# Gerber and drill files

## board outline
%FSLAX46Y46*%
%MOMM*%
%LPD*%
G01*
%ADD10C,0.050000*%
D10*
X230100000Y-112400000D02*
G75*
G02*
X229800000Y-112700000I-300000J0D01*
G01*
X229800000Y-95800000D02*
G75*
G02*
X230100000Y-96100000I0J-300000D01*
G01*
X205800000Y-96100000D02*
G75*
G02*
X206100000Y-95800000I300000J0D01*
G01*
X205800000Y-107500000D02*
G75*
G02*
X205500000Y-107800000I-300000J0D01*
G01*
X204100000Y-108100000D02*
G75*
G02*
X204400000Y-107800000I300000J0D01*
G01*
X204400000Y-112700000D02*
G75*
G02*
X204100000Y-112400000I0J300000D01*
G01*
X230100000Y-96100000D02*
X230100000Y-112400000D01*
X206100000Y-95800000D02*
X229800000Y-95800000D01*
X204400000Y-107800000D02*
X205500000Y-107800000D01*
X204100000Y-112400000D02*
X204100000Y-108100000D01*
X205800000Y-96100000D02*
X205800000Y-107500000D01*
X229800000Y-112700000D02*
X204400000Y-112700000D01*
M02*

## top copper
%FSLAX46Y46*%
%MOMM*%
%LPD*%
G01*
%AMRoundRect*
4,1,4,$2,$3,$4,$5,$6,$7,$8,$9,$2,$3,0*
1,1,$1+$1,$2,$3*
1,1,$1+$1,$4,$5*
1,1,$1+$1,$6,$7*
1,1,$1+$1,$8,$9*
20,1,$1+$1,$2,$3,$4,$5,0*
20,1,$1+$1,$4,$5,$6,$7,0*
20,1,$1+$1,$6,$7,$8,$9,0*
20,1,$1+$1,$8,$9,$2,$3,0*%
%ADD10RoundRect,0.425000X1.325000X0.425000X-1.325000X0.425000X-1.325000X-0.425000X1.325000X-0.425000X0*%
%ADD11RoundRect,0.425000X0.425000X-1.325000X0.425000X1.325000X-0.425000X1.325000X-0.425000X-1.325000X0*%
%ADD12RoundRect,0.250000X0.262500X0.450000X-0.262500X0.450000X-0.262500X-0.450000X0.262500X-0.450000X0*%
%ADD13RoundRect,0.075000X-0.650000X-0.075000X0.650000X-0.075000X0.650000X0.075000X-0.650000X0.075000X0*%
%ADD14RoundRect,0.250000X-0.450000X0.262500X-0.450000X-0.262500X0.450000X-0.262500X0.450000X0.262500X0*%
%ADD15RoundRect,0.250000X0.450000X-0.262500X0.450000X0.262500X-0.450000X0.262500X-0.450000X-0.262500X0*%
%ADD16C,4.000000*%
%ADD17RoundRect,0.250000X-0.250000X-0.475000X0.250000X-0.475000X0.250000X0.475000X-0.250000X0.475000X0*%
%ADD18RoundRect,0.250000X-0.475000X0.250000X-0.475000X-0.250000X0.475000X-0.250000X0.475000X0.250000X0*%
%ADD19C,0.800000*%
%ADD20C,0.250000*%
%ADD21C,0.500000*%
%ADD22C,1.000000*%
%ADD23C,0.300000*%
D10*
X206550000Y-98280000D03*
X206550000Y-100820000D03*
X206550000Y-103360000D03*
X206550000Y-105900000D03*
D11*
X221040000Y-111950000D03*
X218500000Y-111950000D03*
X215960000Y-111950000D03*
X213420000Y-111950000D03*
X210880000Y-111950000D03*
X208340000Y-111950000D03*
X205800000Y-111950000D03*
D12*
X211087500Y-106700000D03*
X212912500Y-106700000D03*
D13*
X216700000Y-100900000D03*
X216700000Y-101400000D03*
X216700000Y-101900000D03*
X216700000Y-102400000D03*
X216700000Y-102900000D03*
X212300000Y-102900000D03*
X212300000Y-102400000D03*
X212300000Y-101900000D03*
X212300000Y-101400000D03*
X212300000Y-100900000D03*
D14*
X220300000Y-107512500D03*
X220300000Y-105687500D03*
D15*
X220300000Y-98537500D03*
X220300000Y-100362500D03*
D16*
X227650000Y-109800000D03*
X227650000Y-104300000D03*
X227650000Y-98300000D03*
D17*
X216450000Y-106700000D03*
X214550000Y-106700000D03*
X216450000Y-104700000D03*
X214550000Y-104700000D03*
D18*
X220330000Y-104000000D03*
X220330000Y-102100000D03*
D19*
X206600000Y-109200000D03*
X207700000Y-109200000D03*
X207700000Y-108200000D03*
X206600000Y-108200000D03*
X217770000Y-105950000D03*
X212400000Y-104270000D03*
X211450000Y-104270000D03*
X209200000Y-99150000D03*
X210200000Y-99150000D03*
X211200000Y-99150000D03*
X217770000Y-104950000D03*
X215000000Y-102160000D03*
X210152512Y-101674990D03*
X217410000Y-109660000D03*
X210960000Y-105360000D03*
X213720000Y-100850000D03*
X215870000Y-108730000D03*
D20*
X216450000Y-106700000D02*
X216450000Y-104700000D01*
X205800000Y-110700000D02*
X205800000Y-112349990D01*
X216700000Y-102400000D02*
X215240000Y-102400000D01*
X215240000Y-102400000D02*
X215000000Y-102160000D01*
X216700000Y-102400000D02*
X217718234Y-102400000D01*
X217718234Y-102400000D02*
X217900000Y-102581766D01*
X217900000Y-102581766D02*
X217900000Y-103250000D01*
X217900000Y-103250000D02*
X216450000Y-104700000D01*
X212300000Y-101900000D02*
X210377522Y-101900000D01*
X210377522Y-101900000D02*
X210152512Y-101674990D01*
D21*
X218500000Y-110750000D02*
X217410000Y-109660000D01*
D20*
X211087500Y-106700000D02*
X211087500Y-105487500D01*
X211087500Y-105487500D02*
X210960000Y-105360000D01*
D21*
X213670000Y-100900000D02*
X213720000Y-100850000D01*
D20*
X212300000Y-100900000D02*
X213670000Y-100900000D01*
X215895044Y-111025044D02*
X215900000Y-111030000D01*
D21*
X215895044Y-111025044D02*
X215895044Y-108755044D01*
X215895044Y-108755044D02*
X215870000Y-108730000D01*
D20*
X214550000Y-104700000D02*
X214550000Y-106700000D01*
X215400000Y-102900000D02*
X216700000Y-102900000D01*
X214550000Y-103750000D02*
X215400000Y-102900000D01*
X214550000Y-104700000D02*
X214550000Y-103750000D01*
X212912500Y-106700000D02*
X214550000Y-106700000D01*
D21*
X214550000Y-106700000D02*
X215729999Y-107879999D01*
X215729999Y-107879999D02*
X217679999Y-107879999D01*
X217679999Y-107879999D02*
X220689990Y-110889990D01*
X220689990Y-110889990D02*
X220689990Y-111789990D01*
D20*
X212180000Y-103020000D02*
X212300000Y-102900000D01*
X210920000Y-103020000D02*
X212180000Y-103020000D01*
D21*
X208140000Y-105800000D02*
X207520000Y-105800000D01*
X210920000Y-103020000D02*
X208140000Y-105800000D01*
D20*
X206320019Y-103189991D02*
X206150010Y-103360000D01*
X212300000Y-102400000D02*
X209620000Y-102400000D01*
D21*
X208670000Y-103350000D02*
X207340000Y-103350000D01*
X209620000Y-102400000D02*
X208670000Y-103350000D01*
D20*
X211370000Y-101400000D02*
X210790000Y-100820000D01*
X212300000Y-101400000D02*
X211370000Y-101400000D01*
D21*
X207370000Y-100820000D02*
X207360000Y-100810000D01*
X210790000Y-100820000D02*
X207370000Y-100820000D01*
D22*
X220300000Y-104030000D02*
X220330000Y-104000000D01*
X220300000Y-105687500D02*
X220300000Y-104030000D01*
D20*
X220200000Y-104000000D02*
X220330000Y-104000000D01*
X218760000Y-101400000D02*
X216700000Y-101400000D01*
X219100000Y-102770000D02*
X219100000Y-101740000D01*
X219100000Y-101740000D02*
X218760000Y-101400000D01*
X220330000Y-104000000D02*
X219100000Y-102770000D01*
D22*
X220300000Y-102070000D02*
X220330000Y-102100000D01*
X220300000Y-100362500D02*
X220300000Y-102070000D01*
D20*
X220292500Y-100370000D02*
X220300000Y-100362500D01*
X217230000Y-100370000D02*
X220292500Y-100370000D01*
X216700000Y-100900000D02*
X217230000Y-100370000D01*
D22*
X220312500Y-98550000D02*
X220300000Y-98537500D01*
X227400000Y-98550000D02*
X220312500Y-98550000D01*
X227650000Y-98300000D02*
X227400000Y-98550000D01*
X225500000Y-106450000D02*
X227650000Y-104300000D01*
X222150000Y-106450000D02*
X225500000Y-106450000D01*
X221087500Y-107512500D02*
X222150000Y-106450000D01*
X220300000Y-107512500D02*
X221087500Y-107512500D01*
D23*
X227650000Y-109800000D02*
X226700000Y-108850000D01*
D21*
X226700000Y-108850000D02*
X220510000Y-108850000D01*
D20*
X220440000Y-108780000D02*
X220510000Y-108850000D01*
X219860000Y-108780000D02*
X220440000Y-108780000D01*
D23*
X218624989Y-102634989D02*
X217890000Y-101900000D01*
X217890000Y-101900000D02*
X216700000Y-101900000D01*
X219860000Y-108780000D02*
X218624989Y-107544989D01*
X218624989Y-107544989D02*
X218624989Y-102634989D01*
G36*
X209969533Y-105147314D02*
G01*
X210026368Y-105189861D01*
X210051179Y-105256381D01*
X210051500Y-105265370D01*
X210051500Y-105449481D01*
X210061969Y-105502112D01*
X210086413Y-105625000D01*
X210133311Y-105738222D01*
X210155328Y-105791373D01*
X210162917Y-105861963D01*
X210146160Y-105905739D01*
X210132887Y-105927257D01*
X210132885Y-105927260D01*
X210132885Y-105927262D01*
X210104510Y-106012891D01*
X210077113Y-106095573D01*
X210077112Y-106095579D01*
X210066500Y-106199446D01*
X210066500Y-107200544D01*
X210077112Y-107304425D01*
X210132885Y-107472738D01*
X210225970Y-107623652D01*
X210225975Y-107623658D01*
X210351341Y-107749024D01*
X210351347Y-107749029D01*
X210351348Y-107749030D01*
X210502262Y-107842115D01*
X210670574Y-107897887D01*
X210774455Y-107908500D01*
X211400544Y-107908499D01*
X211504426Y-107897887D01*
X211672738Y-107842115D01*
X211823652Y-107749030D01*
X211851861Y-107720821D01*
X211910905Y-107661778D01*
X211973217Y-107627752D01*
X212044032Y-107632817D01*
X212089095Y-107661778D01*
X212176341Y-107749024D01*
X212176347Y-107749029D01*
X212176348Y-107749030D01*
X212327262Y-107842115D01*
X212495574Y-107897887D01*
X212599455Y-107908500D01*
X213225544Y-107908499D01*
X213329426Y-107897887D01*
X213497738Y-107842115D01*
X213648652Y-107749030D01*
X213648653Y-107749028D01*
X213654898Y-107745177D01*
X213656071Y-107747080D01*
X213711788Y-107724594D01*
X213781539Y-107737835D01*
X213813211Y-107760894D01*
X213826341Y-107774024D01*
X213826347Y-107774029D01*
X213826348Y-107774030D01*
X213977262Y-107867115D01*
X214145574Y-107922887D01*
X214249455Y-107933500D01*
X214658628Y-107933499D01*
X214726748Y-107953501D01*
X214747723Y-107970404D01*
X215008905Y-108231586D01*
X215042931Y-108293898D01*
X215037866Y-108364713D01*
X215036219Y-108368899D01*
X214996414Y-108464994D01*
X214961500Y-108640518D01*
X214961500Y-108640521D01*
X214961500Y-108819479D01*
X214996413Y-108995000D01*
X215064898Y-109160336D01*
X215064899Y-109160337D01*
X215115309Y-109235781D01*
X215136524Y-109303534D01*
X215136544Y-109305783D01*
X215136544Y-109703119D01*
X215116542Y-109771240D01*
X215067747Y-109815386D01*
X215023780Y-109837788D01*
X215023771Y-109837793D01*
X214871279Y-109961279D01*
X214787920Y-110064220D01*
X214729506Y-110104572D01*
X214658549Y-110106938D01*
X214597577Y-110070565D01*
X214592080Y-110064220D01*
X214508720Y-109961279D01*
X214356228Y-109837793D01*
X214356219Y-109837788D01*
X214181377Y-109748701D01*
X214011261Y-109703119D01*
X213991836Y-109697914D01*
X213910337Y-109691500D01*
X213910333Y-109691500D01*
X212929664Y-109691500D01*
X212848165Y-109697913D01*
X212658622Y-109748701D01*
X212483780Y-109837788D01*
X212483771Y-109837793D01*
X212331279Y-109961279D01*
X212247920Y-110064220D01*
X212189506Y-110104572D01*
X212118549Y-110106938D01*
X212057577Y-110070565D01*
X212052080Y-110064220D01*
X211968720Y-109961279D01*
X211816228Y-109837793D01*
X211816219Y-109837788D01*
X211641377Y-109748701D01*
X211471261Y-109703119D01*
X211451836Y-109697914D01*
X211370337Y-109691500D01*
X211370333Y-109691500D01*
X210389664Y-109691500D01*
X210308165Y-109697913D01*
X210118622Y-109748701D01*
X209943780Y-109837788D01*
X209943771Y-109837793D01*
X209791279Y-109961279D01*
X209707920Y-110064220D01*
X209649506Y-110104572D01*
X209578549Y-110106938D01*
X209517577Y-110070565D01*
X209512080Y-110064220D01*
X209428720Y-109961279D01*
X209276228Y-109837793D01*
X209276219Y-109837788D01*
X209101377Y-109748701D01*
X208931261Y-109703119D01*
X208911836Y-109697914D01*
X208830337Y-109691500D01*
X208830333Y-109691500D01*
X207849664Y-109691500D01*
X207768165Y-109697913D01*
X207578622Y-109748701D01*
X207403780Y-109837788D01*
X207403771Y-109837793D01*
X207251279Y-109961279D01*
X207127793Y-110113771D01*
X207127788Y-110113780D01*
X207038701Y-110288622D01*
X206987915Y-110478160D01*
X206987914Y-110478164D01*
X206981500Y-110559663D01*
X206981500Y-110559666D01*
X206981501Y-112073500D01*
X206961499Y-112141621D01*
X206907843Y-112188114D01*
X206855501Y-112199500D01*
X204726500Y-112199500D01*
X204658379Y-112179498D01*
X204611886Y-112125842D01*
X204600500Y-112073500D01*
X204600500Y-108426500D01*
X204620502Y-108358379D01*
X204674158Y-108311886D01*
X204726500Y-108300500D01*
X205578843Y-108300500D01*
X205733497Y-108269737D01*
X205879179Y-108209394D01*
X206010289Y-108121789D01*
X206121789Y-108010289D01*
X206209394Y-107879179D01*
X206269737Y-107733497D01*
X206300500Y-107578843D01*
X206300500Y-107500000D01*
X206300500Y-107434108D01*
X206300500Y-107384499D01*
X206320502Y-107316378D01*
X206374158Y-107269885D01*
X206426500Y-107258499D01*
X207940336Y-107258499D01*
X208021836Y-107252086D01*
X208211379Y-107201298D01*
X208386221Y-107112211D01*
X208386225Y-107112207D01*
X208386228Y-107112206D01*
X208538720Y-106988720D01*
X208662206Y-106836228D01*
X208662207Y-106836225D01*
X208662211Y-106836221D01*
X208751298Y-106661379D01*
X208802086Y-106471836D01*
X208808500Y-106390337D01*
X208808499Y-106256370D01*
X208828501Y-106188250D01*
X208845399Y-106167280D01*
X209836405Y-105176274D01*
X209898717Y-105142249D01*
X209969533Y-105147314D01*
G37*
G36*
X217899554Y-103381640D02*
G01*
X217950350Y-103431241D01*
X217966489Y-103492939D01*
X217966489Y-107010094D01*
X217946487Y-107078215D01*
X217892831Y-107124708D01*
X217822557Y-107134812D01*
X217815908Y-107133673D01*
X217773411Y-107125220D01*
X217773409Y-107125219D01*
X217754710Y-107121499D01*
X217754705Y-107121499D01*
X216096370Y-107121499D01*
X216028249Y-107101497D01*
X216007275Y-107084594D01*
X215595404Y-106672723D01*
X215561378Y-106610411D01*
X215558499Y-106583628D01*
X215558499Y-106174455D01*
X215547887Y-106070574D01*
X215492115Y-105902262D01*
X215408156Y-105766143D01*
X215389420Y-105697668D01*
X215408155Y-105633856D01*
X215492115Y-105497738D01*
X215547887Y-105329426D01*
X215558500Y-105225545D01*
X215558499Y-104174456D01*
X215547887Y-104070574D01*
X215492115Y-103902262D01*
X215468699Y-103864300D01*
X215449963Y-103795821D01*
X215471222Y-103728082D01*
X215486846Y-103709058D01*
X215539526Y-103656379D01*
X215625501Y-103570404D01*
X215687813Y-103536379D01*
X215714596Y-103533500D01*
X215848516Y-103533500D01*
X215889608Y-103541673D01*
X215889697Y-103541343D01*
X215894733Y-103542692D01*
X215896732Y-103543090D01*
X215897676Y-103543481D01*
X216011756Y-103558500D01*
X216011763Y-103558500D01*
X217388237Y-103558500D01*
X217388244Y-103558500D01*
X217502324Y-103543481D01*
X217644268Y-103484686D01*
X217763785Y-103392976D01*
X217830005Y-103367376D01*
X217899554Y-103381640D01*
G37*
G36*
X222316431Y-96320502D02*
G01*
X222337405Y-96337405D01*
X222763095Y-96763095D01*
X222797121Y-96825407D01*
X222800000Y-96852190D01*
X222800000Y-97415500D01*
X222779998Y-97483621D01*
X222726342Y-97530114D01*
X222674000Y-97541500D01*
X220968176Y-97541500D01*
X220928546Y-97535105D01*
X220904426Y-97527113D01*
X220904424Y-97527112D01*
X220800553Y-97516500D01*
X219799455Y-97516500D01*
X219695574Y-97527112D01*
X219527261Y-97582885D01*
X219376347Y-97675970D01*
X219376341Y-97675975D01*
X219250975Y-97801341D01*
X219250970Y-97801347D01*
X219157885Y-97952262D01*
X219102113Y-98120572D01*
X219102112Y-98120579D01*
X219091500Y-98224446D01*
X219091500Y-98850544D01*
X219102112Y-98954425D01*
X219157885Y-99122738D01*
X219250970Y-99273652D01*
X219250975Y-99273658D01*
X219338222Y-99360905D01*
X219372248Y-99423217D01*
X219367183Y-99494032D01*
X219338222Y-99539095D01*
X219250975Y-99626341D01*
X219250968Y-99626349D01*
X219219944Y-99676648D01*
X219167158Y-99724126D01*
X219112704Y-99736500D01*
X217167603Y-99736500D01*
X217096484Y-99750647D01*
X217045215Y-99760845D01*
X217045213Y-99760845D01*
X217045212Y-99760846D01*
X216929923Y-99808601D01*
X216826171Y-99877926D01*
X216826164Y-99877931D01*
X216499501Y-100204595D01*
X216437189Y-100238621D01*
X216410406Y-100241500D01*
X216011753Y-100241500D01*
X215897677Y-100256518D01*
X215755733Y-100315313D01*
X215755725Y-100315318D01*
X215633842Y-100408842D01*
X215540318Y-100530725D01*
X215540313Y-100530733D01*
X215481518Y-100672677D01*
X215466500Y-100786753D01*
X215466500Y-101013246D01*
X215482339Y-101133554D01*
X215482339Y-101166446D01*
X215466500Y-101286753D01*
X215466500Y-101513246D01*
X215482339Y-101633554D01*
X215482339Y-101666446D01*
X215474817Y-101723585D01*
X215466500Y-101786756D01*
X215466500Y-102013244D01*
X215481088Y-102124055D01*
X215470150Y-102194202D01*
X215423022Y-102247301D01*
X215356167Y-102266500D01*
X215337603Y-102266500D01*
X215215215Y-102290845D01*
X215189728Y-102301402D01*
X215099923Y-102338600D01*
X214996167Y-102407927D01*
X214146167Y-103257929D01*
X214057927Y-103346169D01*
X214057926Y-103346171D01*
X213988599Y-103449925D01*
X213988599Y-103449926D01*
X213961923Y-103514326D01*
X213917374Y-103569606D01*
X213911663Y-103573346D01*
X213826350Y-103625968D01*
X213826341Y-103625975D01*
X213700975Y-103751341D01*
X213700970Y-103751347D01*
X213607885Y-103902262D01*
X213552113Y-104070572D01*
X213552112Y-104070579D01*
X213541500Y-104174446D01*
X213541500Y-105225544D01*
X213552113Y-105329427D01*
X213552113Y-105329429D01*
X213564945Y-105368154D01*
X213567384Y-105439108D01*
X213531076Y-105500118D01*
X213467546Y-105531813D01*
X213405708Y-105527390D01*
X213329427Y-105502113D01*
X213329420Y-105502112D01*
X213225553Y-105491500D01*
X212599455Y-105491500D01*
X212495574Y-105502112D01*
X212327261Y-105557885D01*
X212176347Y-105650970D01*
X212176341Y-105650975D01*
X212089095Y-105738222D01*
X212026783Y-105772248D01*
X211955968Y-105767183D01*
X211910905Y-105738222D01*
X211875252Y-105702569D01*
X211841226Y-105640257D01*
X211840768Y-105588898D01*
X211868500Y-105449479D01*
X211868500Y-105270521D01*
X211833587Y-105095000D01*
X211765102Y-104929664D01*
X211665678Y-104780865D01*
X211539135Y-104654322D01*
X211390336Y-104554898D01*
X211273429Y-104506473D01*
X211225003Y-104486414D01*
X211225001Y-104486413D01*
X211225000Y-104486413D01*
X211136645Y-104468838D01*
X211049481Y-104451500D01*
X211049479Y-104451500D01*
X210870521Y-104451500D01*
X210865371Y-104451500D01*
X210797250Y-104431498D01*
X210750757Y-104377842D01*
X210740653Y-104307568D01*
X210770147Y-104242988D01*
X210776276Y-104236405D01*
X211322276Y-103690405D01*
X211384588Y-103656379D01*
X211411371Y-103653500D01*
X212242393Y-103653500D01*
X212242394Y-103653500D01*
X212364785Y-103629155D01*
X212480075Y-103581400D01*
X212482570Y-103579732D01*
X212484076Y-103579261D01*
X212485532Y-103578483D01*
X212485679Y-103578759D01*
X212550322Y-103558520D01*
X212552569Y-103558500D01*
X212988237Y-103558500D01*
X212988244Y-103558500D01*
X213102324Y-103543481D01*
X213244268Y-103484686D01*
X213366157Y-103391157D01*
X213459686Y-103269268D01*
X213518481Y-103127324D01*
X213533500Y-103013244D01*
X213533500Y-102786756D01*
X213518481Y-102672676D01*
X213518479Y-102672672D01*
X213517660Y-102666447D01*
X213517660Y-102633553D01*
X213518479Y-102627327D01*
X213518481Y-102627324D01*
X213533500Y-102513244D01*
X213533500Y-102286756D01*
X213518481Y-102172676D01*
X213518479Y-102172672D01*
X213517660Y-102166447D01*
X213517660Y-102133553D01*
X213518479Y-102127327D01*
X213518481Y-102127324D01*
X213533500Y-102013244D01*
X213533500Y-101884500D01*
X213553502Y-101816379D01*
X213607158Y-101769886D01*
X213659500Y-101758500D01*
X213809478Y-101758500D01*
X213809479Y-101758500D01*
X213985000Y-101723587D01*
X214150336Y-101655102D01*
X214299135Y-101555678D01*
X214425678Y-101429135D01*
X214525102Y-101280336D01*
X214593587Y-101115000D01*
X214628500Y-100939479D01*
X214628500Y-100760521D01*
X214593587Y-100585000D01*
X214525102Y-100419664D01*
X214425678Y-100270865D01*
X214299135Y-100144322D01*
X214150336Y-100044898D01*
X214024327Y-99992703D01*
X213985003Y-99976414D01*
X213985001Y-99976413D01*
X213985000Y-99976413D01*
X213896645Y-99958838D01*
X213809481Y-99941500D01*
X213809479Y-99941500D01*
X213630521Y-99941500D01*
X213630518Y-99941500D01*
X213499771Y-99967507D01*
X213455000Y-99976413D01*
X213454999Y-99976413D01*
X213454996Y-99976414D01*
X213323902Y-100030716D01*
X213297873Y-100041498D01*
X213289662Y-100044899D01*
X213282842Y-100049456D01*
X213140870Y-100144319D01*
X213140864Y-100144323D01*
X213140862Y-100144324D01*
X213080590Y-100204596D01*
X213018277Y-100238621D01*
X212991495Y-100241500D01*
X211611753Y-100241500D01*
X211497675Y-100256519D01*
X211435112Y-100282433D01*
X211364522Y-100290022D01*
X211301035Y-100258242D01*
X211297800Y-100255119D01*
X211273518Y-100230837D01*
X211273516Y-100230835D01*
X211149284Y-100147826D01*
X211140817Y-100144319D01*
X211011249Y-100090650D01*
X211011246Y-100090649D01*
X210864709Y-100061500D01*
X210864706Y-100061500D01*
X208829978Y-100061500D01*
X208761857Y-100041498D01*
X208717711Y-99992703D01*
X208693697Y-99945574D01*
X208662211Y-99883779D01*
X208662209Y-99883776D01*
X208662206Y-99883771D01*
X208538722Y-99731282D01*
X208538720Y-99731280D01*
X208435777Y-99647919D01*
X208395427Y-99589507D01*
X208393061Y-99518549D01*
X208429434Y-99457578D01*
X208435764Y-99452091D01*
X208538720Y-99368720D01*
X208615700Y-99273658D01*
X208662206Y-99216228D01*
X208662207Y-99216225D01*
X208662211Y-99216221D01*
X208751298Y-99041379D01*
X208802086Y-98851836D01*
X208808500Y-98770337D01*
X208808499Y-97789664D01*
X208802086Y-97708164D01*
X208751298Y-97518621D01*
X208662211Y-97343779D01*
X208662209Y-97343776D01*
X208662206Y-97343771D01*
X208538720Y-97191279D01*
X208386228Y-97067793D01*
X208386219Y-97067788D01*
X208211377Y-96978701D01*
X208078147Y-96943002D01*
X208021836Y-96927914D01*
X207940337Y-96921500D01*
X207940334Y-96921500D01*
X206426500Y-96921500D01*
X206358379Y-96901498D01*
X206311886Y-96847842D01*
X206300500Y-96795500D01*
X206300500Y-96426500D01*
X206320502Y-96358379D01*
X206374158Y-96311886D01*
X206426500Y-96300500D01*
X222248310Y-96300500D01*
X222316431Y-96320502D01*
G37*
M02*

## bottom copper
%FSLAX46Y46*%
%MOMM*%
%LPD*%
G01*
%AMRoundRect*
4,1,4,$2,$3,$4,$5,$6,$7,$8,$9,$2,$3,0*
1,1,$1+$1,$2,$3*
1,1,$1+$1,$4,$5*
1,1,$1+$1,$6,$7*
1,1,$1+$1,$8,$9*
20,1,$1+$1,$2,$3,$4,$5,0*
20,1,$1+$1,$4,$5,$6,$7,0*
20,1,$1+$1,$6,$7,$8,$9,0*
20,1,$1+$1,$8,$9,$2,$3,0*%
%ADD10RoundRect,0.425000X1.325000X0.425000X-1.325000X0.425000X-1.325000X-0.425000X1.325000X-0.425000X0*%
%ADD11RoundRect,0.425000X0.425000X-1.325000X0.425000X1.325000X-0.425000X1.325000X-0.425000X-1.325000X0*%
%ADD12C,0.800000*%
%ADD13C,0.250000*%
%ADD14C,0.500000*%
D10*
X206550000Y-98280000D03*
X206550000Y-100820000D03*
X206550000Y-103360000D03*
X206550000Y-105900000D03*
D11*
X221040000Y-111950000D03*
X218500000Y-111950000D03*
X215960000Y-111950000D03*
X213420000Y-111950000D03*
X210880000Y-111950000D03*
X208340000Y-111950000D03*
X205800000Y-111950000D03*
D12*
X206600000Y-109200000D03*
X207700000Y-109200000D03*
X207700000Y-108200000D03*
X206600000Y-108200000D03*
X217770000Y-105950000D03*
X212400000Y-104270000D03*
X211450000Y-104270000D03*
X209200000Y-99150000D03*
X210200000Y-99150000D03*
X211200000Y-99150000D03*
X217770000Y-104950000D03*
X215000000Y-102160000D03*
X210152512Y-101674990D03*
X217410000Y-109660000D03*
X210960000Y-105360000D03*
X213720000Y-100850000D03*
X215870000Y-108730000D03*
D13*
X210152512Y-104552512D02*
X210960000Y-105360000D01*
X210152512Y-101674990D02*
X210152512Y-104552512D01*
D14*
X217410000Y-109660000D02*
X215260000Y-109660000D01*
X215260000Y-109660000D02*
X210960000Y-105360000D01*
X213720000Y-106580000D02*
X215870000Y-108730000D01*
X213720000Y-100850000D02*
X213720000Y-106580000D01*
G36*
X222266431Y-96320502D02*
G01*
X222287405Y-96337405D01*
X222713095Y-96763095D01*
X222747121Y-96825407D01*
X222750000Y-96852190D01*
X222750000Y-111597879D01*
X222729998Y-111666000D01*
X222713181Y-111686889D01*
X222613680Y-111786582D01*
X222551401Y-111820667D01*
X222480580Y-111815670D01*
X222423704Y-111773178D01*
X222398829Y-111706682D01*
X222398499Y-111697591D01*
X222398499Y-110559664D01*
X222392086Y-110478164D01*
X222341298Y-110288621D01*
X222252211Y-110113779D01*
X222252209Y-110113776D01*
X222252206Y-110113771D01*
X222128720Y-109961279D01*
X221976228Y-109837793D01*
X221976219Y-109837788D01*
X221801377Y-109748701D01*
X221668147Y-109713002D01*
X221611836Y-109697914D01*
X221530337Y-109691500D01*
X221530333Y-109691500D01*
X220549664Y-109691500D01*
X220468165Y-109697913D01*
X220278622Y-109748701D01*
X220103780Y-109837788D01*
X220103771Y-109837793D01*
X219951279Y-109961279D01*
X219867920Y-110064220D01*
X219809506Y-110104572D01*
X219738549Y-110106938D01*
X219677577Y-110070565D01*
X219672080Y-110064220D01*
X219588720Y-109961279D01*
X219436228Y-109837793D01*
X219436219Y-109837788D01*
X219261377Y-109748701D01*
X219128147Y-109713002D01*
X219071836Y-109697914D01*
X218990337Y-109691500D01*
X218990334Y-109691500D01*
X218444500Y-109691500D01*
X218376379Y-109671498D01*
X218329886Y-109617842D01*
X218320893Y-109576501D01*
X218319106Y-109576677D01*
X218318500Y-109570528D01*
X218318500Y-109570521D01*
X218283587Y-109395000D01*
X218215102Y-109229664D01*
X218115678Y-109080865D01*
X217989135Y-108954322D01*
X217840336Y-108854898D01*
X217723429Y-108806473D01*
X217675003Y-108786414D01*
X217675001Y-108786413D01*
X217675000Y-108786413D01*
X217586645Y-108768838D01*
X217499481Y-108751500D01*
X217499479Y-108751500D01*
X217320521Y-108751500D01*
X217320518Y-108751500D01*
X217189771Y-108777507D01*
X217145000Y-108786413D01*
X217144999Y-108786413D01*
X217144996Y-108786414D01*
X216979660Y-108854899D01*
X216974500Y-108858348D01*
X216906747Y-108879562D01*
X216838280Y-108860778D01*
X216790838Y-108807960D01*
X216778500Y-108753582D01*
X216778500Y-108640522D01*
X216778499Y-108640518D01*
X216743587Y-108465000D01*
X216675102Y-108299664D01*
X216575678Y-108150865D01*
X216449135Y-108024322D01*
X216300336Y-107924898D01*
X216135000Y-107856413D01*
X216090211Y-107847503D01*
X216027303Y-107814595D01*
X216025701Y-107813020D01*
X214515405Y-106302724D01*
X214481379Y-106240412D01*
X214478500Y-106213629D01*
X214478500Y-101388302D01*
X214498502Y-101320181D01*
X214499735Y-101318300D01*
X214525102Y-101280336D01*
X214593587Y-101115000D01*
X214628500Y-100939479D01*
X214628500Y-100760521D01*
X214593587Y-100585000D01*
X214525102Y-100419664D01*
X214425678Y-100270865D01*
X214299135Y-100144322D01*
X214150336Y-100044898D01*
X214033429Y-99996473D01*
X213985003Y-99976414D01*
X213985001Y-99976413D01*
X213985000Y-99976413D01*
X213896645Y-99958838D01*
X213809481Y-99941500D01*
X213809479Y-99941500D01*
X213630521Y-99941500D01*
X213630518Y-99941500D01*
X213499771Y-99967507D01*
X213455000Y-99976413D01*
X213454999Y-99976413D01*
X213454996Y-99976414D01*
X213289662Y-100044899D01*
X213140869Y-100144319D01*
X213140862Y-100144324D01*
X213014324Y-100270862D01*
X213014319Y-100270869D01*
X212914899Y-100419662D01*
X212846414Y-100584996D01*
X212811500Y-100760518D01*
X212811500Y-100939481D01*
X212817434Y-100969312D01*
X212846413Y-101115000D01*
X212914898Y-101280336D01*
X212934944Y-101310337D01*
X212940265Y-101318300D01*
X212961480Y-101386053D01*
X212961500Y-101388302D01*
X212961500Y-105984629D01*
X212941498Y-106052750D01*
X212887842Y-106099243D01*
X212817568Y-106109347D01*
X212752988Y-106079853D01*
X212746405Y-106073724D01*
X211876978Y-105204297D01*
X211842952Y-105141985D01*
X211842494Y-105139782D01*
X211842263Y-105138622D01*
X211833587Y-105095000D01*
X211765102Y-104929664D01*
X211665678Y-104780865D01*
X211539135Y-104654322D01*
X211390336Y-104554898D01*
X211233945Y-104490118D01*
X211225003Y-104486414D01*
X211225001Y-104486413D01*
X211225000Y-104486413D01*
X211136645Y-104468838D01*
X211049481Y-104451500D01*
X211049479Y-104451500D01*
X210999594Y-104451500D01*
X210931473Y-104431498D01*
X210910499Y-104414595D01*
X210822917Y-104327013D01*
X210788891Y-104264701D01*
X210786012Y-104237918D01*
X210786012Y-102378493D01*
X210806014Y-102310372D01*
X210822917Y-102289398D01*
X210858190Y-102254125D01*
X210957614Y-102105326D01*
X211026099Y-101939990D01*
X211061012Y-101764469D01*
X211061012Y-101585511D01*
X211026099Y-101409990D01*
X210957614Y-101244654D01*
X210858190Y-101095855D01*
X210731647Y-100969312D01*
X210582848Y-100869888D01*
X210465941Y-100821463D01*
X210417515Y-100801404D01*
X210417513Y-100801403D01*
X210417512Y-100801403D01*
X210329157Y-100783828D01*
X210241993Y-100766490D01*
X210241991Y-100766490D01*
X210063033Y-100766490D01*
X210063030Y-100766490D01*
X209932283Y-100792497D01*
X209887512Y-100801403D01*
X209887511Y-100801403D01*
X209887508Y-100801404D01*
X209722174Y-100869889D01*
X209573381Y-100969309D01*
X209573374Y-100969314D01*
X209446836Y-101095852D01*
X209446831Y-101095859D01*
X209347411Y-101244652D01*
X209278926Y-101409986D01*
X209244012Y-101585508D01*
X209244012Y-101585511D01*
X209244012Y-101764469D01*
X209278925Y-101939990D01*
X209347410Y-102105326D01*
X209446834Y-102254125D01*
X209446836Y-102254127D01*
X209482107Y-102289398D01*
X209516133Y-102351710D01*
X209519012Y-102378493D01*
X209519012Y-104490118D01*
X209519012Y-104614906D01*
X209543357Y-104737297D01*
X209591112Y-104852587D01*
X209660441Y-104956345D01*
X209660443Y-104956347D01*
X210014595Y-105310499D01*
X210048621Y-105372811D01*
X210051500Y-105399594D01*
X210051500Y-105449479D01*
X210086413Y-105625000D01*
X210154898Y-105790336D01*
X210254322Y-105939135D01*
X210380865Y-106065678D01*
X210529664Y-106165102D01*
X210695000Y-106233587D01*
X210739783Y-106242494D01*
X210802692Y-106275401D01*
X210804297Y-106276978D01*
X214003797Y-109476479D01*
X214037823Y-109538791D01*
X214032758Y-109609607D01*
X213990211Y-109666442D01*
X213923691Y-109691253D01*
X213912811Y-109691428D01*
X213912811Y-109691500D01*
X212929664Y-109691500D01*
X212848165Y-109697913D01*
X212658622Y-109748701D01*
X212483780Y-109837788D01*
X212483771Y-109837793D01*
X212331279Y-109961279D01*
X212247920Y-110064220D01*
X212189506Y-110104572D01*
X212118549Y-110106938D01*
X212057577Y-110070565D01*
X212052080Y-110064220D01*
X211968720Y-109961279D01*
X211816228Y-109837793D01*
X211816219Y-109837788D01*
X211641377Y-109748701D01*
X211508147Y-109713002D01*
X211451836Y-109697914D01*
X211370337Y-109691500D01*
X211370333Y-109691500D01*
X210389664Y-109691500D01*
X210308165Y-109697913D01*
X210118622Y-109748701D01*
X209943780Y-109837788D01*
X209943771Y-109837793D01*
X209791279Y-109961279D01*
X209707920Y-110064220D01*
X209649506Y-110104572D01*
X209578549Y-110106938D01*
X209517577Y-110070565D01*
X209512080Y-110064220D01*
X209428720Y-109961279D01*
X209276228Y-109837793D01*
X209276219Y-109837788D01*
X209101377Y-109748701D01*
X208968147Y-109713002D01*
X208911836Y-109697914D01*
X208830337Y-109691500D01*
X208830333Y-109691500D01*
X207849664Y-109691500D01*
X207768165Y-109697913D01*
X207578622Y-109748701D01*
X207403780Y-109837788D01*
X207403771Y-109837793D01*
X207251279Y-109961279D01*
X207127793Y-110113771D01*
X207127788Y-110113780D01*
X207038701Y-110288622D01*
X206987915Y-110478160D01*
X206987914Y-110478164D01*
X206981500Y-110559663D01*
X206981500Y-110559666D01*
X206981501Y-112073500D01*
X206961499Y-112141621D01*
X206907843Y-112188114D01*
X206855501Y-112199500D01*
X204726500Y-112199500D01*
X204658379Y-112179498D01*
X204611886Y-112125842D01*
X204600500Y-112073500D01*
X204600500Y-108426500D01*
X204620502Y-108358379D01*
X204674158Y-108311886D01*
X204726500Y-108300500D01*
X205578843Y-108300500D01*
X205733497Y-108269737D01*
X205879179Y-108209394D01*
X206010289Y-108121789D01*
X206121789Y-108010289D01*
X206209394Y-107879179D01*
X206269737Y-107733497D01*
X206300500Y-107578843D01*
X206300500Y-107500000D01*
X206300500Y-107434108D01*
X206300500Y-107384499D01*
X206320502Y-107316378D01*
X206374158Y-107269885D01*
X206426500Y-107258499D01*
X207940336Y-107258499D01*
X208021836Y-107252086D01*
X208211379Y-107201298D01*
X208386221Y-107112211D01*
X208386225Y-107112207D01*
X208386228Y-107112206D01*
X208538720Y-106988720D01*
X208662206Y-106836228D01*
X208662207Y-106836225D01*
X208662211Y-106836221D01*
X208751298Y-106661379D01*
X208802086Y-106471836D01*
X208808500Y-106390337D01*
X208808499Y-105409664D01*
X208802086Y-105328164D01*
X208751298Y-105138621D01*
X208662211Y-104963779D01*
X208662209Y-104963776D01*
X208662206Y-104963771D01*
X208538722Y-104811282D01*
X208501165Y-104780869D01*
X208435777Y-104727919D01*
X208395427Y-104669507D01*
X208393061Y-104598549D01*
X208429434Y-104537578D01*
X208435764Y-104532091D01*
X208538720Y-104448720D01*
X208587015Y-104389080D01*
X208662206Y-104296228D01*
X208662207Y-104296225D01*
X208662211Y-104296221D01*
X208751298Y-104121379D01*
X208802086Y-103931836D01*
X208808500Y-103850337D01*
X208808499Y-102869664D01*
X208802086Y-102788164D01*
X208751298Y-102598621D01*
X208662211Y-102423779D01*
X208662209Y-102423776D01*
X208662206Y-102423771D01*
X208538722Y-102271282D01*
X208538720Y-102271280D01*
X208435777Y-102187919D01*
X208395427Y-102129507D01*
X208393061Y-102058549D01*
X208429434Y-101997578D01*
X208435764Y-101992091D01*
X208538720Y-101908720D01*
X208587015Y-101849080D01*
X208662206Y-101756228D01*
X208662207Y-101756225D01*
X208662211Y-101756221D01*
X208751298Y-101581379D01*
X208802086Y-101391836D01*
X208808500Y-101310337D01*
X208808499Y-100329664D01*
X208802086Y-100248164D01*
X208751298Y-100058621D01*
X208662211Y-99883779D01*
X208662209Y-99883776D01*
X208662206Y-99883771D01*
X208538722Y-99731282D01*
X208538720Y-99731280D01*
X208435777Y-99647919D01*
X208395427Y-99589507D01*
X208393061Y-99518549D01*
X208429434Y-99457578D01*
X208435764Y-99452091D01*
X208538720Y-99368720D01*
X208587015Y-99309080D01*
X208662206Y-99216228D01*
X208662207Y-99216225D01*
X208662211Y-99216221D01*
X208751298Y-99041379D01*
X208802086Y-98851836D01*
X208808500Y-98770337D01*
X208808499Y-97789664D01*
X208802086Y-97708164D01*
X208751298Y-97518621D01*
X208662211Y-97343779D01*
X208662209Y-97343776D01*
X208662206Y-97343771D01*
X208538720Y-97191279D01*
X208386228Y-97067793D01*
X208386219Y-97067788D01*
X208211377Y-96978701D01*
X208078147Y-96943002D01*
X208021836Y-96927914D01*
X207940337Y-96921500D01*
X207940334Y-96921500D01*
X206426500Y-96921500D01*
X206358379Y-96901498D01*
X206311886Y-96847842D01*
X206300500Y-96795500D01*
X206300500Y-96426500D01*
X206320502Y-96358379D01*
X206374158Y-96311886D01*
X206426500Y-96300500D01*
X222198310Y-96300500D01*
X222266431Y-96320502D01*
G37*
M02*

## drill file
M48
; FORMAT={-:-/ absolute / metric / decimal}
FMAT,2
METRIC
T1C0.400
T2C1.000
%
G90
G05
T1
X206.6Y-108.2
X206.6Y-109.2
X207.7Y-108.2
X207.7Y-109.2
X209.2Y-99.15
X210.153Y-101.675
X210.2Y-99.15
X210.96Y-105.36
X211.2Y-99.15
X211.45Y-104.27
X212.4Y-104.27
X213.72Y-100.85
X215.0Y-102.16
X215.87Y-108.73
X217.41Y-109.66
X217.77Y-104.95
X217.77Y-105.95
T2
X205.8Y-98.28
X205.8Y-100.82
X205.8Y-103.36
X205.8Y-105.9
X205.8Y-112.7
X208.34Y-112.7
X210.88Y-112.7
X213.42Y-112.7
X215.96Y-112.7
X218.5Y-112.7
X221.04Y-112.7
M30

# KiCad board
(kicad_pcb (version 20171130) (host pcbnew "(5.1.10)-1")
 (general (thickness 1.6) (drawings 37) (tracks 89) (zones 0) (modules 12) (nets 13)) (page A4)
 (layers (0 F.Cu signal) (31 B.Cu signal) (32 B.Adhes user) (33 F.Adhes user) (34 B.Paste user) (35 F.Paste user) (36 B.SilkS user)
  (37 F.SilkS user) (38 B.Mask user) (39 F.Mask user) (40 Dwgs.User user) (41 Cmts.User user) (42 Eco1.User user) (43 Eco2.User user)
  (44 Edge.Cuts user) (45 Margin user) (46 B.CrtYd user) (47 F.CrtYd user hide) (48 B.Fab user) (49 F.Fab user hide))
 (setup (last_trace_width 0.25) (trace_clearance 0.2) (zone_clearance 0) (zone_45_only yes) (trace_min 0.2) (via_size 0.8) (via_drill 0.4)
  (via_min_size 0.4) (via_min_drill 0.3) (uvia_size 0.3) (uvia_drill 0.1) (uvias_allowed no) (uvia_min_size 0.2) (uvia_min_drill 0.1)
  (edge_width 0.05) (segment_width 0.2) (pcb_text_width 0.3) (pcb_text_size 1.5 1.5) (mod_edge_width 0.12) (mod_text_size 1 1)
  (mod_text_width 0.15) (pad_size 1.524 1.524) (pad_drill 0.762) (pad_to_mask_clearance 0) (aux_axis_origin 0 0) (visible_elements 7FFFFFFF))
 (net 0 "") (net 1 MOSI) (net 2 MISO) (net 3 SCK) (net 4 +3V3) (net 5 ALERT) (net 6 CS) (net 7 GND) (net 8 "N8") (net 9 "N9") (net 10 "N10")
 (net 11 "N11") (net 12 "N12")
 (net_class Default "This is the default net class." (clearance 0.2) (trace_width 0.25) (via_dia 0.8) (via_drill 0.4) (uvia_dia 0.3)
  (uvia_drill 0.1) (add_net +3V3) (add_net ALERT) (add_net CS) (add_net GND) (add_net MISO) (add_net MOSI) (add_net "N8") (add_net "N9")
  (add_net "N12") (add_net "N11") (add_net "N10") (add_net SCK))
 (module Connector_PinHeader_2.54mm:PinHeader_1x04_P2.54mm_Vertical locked (layer F.Cu) (at 205.8 105.9 180)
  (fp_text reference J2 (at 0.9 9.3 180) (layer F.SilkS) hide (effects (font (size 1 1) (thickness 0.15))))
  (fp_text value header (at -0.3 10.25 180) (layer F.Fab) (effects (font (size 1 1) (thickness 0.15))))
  (pad 4 thru_hole roundrect (at 0 7.62 180) (size 3.5 1.7) (drill 1 (offset -0.75 0)) (layers *.Cu *.Mask) (roundrect_rratio 0.25))
  (pad 3 thru_hole roundrect (at 0 5.08 180) (size 3.5 1.7) (drill 1 (offset -0.75 0)) (layers *.Cu *.Mask) (roundrect_rratio 0.25)
   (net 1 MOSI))
  (pad 2 thru_hole roundrect (at 0 2.54 180) (size 3.5 1.7) (drill 1 (offset -0.75 0)) (layers *.Cu *.Mask) (roundrect_rratio 0.25)
   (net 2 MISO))
  (pad 1 thru_hole roundrect (at 0 0 180) (size 3.5 1.7) (drill 1 (offset -0.75 0)) (layers *.Cu *.Mask) (roundrect_rratio 0.25) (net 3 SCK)))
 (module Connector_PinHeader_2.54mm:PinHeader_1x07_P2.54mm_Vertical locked (layer F.Cu) (at 205.8 112.7 90)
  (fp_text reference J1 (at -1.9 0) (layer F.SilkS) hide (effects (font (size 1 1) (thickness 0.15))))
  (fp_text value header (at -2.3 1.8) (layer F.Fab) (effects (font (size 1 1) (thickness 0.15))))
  (pad 7 thru_hole roundrect (at 0 15.24 90) (size 3.5 1.7) (drill 1 (offset 0.75 0)) (layers *.Cu *.Mask) (roundrect_rratio 0.25)
   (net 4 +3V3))
  (pad 6 thru_hole roundrect (at 0 12.7 90) (size 3.5 1.7) (drill 1 (offset 0.75 0)) (layers *.Cu *.Mask) (roundrect_rratio 0.25)
   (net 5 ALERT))
  (pad 5 thru_hole roundrect (at 0 10.16 90) (size 3.5 1.7) (drill 1 (offset 0.75 0)) (layers *.Cu *.Mask) (roundrect_rratio 0.25)
   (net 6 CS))
  (pad 4 thru_hole roundrect (at 0 7.62 90) (size 3.5 1.7) (drill 1 (offset 0.75 0)) (layers *.Cu *.Mask) (roundrect_rratio 0.25))
  (pad 3 thru_hole roundrect (at 0 5.08 90) (size 3.5 1.7) (drill 1 (offset 0.75 0)) (layers *.Cu *.Mask) (roundrect_rratio 0.25))
  (pad 2 thru_hole roundrect (at 0 2.54 90) (size 3.5 1.7) (drill 1 (offset 0.75 0)) (layers *.Cu *.Mask) (roundrect_rratio 0.25))
  (pad 1 thru_hole roundrect (at 0 0 90) (size 3.5 1.7) (drill 1 (offset 0.75 0)) (layers *.Cu *.Mask) (roundrect_rratio 0.25) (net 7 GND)))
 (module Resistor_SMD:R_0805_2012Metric (layer F.Cu) (at 212 106.7 180)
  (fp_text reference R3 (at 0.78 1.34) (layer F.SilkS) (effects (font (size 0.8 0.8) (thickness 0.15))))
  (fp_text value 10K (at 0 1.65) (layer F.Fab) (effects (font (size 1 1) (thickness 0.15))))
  (pad 2 smd roundrect (at 0.9125 0 180) (size 1.025 1.4) (layers F.Cu F.Paste F.Mask) (roundrect_rratio 0.243902) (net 5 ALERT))
  (pad 1 smd roundrect (at -0.9125 0 180) (size 1.025 1.4) (layers F.Cu F.Paste F.Mask) (roundrect_rratio 0.243902) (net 4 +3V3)))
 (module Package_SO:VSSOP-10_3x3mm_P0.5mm (layer F.Cu) (at 214.5 101.9)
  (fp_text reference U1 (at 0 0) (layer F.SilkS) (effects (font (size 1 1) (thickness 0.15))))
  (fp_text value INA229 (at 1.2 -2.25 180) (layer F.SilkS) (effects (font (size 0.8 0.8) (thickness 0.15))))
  (pad 10 smd roundrect (at 2.2 -1) (size 1.45 0.3) (layers F.Cu F.Paste F.Mask) (roundrect_rratio 0.25) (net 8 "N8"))
  (pad 9 smd roundrect (at 2.2 -0.5) (size 1.45 0.3) (layers F.Cu F.Paste F.Mask) (roundrect_rratio 0.25) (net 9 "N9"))
  (pad 8 smd roundrect (at 2.2 0) (size 1.45 0.3) (layers F.Cu F.Paste F.Mask) (roundrect_rratio 0.25) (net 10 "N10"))
  (pad 7 smd roundrect (at 2.2 0.5) (size 1.45 0.3) (layers F.Cu F.Paste F.Mask) (roundrect_rratio 0.25) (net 7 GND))
  (pad 6 smd roundrect (at 2.2 1) (size 1.45 0.3) (layers F.Cu F.Paste F.Mask) (roundrect_rratio 0.25) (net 4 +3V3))
  (pad 5 smd roundrect (at -2.2 1) (size 1.45 0.3) (layers F.Cu F.Paste F.Mask) (roundrect_rratio 0.25) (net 3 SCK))
  (pad 4 smd roundrect (at -2.2 0.5) (size 1.45 0.3) (layers F.Cu F.Paste F.Mask) (roundrect_rratio 0.25) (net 2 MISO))
  (pad 3 smd roundrect (at -2.2 0) (size 1.45 0.3) (layers F.Cu F.Paste F.Mask) (roundrect_rratio 0.25) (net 5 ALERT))
  (pad 2 smd roundrect (at -2.2 -0.5) (size 1.45 0.3) (layers F.Cu F.Paste F.Mask) (roundrect_rratio 0.25) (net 1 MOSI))
  (pad 1 smd roundrect (at -2.2 -1) (size 1.45 0.3) (layers F.Cu F.Paste F.Mask) (roundrect_rratio 0.25) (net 6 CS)))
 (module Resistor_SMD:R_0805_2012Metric (layer F.Cu) (at 220.3 106.6 270)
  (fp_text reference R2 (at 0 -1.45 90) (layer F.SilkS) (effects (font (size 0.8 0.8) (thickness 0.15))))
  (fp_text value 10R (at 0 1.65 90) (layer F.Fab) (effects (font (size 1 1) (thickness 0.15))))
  (pad 2 smd roundrect (at 0.9125 0 270) (size 1.025 1.4) (layers F.Cu F.Paste F.Mask) (roundrect_rratio 0.243902) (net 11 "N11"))
  (pad 1 smd roundrect (at -0.9125 0 270) (size 1.025 1.4) (layers F.Cu F.Paste F.Mask) (roundrect_rratio 0.243902) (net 9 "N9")))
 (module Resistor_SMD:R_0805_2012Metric (layer F.Cu) (at 220.3 99.45 90)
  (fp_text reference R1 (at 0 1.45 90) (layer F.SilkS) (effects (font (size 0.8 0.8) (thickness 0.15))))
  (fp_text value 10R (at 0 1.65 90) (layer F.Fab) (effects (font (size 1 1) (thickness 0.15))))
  (pad 2 smd roundrect (at 0.9125 0 90) (size 1.025 1.4) (layers F.Cu F.Paste F.Mask) (roundrect_rratio 0.243902) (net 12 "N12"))
  (pad 1 smd roundrect (at -0.9125 0 90) (size 1.025 1.4) (layers F.Cu F.Paste F.Mask) (roundrect_rratio 0.243902) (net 8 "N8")))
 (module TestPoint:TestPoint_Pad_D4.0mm (layer F.Cu) (at 227.65 109.8 90)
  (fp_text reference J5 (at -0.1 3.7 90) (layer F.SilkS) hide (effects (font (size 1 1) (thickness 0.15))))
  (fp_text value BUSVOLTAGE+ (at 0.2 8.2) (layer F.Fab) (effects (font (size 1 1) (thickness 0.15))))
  (pad 1 smd circle (at 0 0 90) (size 4 4) (layers F.Cu F.Mask) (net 10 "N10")))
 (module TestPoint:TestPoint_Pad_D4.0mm (layer F.Cu) (at 227.65 104.3 90)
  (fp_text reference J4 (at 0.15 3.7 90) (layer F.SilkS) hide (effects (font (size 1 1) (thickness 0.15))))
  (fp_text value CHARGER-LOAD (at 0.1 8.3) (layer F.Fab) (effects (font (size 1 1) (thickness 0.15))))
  (pad 1 smd circle (at 0 0 90) (size 4 4) (layers F.Cu F.Mask) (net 11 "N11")))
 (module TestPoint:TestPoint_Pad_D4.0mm (layer F.Cu) (at 227.65 98.3 90)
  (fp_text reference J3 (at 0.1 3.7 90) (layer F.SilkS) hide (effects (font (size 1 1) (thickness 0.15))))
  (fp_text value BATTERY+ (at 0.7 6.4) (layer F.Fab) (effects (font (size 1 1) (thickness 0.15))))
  (pad 1 smd circle (at 0 0 90) (size 4 4) (layers F.Cu F.Mask) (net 12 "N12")))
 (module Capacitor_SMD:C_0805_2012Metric (layer F.Cu) (at 215.5 106.7)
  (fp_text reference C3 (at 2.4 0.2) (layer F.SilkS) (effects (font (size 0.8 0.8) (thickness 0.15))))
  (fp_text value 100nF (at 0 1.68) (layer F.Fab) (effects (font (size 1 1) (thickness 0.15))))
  (pad 2 smd roundrect (at 0.95 0) (size 1 1.45) (layers F.Cu F.Paste F.Mask) (roundrect_rratio 0.25) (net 7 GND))
  (pad 1 smd roundrect (at -0.95 0) (size 1 1.45) (layers F.Cu F.Paste F.Mask) (roundrect_rratio 0.25) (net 4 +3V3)))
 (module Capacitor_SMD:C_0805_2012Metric (layer F.Cu) (at 215.5 104.7)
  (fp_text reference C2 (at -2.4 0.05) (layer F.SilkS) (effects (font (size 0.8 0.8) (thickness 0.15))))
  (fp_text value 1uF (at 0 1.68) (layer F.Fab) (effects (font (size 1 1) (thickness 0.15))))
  (pad 2 smd roundrect (at 0.95 0) (size 1 1.45) (layers F.Cu F.Paste F.Mask) (roundrect_rratio 0.25) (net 7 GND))
  (pad 1 smd roundrect (at -0.95 0) (size 1 1.45) (layers F.Cu F.Paste F.Mask) (roundrect_rratio 0.25) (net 4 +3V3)))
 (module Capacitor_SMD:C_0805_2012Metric (layer F.Cu) (at 220.33 103.05 270)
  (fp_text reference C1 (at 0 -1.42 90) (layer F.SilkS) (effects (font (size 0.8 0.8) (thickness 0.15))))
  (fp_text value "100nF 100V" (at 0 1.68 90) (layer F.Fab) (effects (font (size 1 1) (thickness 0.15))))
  (pad 2 smd roundrect (at 0.95 0 270) (size 1 1.45) (layers F.Cu F.Paste F.Mask) (roundrect_rratio 0.25) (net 9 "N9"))
  (pad 1 smd roundrect (at -0.95 0 270) (size 1 1.45) (layers F.Cu F.Paste F.Mask) (roundrect_rratio 0.25) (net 8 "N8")))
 (gr_arc (start 229.8 112.4) (end 229.8 112.7) (angle -90) (layer Edge.Cuts) (width 0.05))
 (gr_arc (start 229.8 96.1) (end 230.1 96.1) (angle -90) (layer Edge.Cuts) (width 0.05))
 (gr_arc (start 206.1 96.1) (end 206.1 95.8) (angle -90) (layer Edge.Cuts) (width 0.05))
 (gr_arc (start 205.5 107.5) (end 205.5 107.8) (angle -90) (layer Edge.Cuts) (width 0.05))
 (gr_arc (start 204.4 108.1) (end 204.4 107.8) (angle -90) (layer Edge.Cuts) (width 0.05))
 (gr_arc (start 204.4 112.4) (end 204.1 112.4) (angle -90) (layer Edge.Cuts) (width 0.05))
 (gr_line (start 230.1 96.1) (end 230.1 112.4) (layer Edge.Cuts) (width 0.05))
 (gr_line (start 206.1 95.8) (end 229.8 95.8) (layer Edge.Cuts) (width 0.05))
 (gr_line (start 204.4 107.8) (end 205.5 107.8) (layer Edge.Cuts) (width 0.05))
 (gr_line (start 204.1 112.4) (end 204.1 108.1) (layer Edge.Cuts) (width 0.05))
 (gr_line (start 205.8 96.1) (end 205.8 107.5) (layer Edge.Cuts) (width 0.05))
 (gr_line (start 229.8 112.7) (end 204.4 112.7) (layer Edge.Cuts) (width 0.05))
 (via (at 206.6 109.2) (size 0.8) (drill 0.4) (layers F.Cu B.Cu) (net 7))
 (segment (start 216.45 106.7) (end 216.45 104.7) (width 0.25) (layer F.Cu) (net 7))
 (segment (start 205.8 110.7) (end 205.8 112.34999) (width 0.25) (layer F.Cu) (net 7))
 (via (at 207.7 109.2) (size 0.8) (drill 0.4) (layers F.Cu B.Cu) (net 7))
 (via (at 207.7 108.2) (size 0.8) (drill 0.4) (layers F.Cu B.Cu) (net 7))
 (via (at 206.6 108.2) (size 0.8) (drill 0.4) (layers F.Cu B.Cu) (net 7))
 (via (at 217.77 105.95) (size 0.8) (drill 0.4) (layers F.Cu B.Cu) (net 7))
 (via (at 212.4 104.27) (size 0.8) (drill 0.4) (layers F.Cu B.Cu) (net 7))
 (via (at 211.45 104.27) (size 0.8) (drill 0.4) (layers F.Cu B.Cu) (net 7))
 (via (at 209.2 99.15) (size 0.8) (drill 0.4) (layers F.Cu B.Cu) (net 7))
 (via (at 210.2 99.15) (size 0.8) (drill 0.4) (layers F.Cu B.Cu) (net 7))
 (via (at 211.2 99.15) (size 0.8) (drill 0.4) (layers F.Cu B.Cu) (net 7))
 (via (at 217.77 104.95) (size 0.8) (drill 0.4) (layers F.Cu B.Cu) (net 7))
 (via (at 215 102.16) (size 0.8) (drill 0.4) (layers F.Cu B.Cu) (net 7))
 (segment (start 216.7 102.4) (end 215.24 102.4) (width 0.25) (layer F.Cu) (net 7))
 (segment (start 215.24 102.4) (end 215 102.16) (width 0.25) (layer F.Cu) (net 7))
 (segment (start 216.7 102.4) (end 217.718234 102.4) (width 0.25) (layer F.Cu) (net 7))
 (segment (start 217.718234 102.4) (end 217.9 102.581766) (width 0.25) (layer F.Cu) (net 7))
 (segment (start 217.9 102.581766) (end 217.9 103.25) (width 0.25) (layer F.Cu) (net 7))
 (segment (start 217.9 103.25) (end 216.45 104.7) (width 0.25) (layer F.Cu) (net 7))
 (via (at 210.152512 101.67499) (size 0.8) (drill 0.4) (layers F.Cu B.Cu) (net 5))
 (segment (start 212.3 101.9) (end 210.377522 101.9) (width 0.25) (layer F.Cu) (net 5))
 (segment (start 210.377522 101.9) (end 210.152512 101.67499) (width 0.25) (layer F.Cu) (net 5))
 (via (at 217.41 109.66) (size 0.8) (drill 0.4) (layers F.Cu B.Cu) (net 5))
 (segment (start 218.5 110.75) (end 217.41 109.66) (width 0.5) (layer F.Cu) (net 5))
 (via (at 210.96 105.36) (size 0.8) (drill 0.4) (layers F.Cu B.Cu) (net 5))
 (segment (start 210.152512 104.552512) (end 210.96 105.36) (width 0.25) (layer B.Cu) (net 5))
 (segment (start 211.0875 106.7) (end 211.0875 105.4875) (width 0.25) (layer F.Cu) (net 5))
 (segment (start 210.152512 101.67499) (end 210.152512 104.552512) (width 0.25) (layer B.Cu) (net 5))
 (segment (start 211.0875 105.4875) (end 210.96 105.36) (width 0.25) (layer F.Cu) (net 5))
 (segment (start 217.41 109.66) (end 215.26 109.66) (width 0.5) (layer B.Cu) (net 5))
 (segment (start 215.26 109.66) (end 210.96 105.36) (width 0.5) (layer B.Cu) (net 5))
 (segment (start 213.67 100.9) (end 213.72 100.85) (width 0.5) (layer F.Cu) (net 6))
 (segment (start 212.3 100.9) (end 213.67 100.9) (width 0.25) (layer F.Cu) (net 6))
 (via (at 213.72 100.85) (size 0.8) (drill 0.4) (layers F.Cu B.Cu) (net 6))
 (segment (start 215.895044 111.025044) (end 215.9 111.03) (width 0.25) (layer F.Cu) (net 6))
 (via (at 215.87 108.73) (size 0.8) (drill 0.4) (layers F.Cu B.Cu) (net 6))
 (segment (start 213.72 106.58) (end 215.87 108.73) (width 0.5) (layer B.Cu) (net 6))
 (segment (start 213.72 100.85) (end 213.72 106.58) (width 0.5) (layer B.Cu) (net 6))
 (segment (start 215.895044 111.025044) (end 215.895044 108.755044) (width 0.5) (layer F.Cu) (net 6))
 (segment (start 215.895044 108.755044) (end 215.87 108.73) (width 0.5) (layer F.Cu) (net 6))
 (segment (start 214.55 104.7) (end 214.55 106.7) (width 0.25) (layer F.Cu) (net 4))
 (segment (start 215.4 102.9) (end 216.7 102.9) (width 0.25) (layer F.Cu) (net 4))
 (segment (start 214.55 103.75) (end 215.4 102.9) (width 0.25) (layer F.Cu) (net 4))
 (segment (start 214.55 104.7) (end 214.55 103.75) (width 0.25) (layer F.Cu) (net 4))
 (segment (start 212.9125 106.7) (end 214.55 106.7) (width 0.25) (layer F.Cu) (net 4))
 (segment (start 214.55 106.7) (end 215.729999 107.879999) (width 0.5) (layer F.Cu) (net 4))
 (segment (start 215.729999 107.879999) (end 217.679999 107.879999) (width 0.5) (layer F.Cu) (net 4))
 (segment (start 217.679999 107.879999) (end 220.68999 110.88999) (width 0.5) (layer F.Cu) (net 4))
 (segment (start 220.68999 110.88999) (end 220.68999 111.78999) (width 0.5) (layer F.Cu) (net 4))
 (segment (start 212.18 103.02) (end 212.3 102.9) (width 0.25) (layer F.Cu) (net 3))
 (segment (start 210.92 103.02) (end 212.18 103.02) (width 0.25) (layer F.Cu) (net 3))
 (segment (start 208.14 105.8) (end 207.52 105.8) (width 0.5) (layer F.Cu) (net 3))
 (segment (start 210.92 103.02) (end 208.14 105.8) (width 0.5) (layer F.Cu) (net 3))
 (segment (start 206.320019 103.189991) (end 206.15001 103.36) (width 0.25) (layer F.Cu) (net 2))
 (segment (start 212.3 102.4) (end 209.62 102.4) (width 0.25) (layer F.Cu) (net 2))
 (segment (start 208.67 103.35) (end 207.34 103.35) (width 0.5) (layer F.Cu) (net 2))
 (segment (start 209.62 102.4) (end 208.67 103.35) (width 0.5) (layer F.Cu) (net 2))
 (segment (start 211.37 101.4) (end 210.79 100.82) (width 0.25) (layer F.Cu) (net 1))
 (segment (start 212.3 101.4) (end 211.37 101.4) (width 0.25) (layer F.Cu) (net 1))
 (segment (start 207.37 100.82) (end 207.36 100.81) (width 0.5) (layer F.Cu) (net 1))
 (segment (start 210.79 100.82) (end 207.37 100.82) (width 0.5) (layer F.Cu) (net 1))
 (segment (start 220.3 104.03) (end 220.33 104) (width 1) (layer F.Cu) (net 9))
 (segment (start 220.3 105.6875) (end 220.3 104.03) (width 1) (layer F.Cu) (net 9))
 (segment (start 220.2 104) (end 220.33 104) (width 0.25) (layer F.Cu) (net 9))
 (segment (start 218.76 101.4) (end 216.7 101.4) (width 0.25) (layer F.Cu) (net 9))
 (segment (start 219.1 102.77) (end 219.1 101.74) (width 0.25) (layer F.Cu) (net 9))
 (segment (start 219.1 101.74) (end 218.76 101.4) (width 0.25) (layer F.Cu) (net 9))
 (segment (start 220.33 104) (end 219.1 102.77) (width 0.25) (layer F.Cu) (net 9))
 (segment (start 220.3 102.07) (end 220.33 102.1) (width 1) (layer F.Cu) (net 8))
 (segment (start 220.3 100.3625) (end 220.3 102.07) (width 1) (layer F.Cu) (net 8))
 (segment (start 220.2925 100.37) (end 220.3 100.3625) (width 0.25) (layer F.Cu) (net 8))
 (segment (start 217.23 100.37) (end 220.2925 100.37) (width 0.25) (layer F.Cu) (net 8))
 (segment (start 216.7 100.9) (end 217.23 100.37) (width 0.25) (layer F.Cu) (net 8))
 (segment (start 220.3125 98.55) (end 220.3 98.5375) (width 1) (layer F.Cu) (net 12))
 (segment (start 227.4 98.55) (end 220.3125 98.55) (width 1) (layer F.Cu) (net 12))
 (segment (start 227.65 98.3) (end 227.4 98.55) (width 1) (layer F.Cu) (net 12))
 (segment (start 225.5 106.45) (end 227.65 104.3) (width 1) (layer F.Cu) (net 11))
 (segment (start 222.15 106.45) (end 225.5 106.45) (width 1) (layer F.Cu) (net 11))
 (segment (start 221.0875 107.5125) (end 222.15 106.45) (width 1) (layer F.Cu) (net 11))
 (segment (start 220.3 107.5125) (end 221.0875 107.5125) (width 1) (layer F.Cu) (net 11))
 (segment (start 227.65 109.8) (end 226.7 108.85) (width 0.3) (layer F.Cu) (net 10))
 (segment (start 226.7 108.85) (end 220.51 108.85) (width 0.5) (layer F.Cu) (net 10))
 (segment (start 220.44 108.78) (end 220.51 108.85) (width 0.25) (layer F.Cu) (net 10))
 (segment (start 219.86 108.78) (end 220.44 108.78) (width 0.25) (layer F.Cu) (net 10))
 (segment (start 218.624989 102.634989) (end 217.89 101.9) (width 0.3) (layer F.Cu) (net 10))
 (segment (start 217.89 101.9) (end 216.7 101.9) (width 0.3) (layer F.Cu) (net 10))
 (segment (start 219.86 108.78) (end 218.624989 107.544989) (width 0.3) (layer F.Cu) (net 10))
 (segment (start 218.624989 107.544989) (end 218.624989 102.634989) (width 0.3) (layer F.Cu) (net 10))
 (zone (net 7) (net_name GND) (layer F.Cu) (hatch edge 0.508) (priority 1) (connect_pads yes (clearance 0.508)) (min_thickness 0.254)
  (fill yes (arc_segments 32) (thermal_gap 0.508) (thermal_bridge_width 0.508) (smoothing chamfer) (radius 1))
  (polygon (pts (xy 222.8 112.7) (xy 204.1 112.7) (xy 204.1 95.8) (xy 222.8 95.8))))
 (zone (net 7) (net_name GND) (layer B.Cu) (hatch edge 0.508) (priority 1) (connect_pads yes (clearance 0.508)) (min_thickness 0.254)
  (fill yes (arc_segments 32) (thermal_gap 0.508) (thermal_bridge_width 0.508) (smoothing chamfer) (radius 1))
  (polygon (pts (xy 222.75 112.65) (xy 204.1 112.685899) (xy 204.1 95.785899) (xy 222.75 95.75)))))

